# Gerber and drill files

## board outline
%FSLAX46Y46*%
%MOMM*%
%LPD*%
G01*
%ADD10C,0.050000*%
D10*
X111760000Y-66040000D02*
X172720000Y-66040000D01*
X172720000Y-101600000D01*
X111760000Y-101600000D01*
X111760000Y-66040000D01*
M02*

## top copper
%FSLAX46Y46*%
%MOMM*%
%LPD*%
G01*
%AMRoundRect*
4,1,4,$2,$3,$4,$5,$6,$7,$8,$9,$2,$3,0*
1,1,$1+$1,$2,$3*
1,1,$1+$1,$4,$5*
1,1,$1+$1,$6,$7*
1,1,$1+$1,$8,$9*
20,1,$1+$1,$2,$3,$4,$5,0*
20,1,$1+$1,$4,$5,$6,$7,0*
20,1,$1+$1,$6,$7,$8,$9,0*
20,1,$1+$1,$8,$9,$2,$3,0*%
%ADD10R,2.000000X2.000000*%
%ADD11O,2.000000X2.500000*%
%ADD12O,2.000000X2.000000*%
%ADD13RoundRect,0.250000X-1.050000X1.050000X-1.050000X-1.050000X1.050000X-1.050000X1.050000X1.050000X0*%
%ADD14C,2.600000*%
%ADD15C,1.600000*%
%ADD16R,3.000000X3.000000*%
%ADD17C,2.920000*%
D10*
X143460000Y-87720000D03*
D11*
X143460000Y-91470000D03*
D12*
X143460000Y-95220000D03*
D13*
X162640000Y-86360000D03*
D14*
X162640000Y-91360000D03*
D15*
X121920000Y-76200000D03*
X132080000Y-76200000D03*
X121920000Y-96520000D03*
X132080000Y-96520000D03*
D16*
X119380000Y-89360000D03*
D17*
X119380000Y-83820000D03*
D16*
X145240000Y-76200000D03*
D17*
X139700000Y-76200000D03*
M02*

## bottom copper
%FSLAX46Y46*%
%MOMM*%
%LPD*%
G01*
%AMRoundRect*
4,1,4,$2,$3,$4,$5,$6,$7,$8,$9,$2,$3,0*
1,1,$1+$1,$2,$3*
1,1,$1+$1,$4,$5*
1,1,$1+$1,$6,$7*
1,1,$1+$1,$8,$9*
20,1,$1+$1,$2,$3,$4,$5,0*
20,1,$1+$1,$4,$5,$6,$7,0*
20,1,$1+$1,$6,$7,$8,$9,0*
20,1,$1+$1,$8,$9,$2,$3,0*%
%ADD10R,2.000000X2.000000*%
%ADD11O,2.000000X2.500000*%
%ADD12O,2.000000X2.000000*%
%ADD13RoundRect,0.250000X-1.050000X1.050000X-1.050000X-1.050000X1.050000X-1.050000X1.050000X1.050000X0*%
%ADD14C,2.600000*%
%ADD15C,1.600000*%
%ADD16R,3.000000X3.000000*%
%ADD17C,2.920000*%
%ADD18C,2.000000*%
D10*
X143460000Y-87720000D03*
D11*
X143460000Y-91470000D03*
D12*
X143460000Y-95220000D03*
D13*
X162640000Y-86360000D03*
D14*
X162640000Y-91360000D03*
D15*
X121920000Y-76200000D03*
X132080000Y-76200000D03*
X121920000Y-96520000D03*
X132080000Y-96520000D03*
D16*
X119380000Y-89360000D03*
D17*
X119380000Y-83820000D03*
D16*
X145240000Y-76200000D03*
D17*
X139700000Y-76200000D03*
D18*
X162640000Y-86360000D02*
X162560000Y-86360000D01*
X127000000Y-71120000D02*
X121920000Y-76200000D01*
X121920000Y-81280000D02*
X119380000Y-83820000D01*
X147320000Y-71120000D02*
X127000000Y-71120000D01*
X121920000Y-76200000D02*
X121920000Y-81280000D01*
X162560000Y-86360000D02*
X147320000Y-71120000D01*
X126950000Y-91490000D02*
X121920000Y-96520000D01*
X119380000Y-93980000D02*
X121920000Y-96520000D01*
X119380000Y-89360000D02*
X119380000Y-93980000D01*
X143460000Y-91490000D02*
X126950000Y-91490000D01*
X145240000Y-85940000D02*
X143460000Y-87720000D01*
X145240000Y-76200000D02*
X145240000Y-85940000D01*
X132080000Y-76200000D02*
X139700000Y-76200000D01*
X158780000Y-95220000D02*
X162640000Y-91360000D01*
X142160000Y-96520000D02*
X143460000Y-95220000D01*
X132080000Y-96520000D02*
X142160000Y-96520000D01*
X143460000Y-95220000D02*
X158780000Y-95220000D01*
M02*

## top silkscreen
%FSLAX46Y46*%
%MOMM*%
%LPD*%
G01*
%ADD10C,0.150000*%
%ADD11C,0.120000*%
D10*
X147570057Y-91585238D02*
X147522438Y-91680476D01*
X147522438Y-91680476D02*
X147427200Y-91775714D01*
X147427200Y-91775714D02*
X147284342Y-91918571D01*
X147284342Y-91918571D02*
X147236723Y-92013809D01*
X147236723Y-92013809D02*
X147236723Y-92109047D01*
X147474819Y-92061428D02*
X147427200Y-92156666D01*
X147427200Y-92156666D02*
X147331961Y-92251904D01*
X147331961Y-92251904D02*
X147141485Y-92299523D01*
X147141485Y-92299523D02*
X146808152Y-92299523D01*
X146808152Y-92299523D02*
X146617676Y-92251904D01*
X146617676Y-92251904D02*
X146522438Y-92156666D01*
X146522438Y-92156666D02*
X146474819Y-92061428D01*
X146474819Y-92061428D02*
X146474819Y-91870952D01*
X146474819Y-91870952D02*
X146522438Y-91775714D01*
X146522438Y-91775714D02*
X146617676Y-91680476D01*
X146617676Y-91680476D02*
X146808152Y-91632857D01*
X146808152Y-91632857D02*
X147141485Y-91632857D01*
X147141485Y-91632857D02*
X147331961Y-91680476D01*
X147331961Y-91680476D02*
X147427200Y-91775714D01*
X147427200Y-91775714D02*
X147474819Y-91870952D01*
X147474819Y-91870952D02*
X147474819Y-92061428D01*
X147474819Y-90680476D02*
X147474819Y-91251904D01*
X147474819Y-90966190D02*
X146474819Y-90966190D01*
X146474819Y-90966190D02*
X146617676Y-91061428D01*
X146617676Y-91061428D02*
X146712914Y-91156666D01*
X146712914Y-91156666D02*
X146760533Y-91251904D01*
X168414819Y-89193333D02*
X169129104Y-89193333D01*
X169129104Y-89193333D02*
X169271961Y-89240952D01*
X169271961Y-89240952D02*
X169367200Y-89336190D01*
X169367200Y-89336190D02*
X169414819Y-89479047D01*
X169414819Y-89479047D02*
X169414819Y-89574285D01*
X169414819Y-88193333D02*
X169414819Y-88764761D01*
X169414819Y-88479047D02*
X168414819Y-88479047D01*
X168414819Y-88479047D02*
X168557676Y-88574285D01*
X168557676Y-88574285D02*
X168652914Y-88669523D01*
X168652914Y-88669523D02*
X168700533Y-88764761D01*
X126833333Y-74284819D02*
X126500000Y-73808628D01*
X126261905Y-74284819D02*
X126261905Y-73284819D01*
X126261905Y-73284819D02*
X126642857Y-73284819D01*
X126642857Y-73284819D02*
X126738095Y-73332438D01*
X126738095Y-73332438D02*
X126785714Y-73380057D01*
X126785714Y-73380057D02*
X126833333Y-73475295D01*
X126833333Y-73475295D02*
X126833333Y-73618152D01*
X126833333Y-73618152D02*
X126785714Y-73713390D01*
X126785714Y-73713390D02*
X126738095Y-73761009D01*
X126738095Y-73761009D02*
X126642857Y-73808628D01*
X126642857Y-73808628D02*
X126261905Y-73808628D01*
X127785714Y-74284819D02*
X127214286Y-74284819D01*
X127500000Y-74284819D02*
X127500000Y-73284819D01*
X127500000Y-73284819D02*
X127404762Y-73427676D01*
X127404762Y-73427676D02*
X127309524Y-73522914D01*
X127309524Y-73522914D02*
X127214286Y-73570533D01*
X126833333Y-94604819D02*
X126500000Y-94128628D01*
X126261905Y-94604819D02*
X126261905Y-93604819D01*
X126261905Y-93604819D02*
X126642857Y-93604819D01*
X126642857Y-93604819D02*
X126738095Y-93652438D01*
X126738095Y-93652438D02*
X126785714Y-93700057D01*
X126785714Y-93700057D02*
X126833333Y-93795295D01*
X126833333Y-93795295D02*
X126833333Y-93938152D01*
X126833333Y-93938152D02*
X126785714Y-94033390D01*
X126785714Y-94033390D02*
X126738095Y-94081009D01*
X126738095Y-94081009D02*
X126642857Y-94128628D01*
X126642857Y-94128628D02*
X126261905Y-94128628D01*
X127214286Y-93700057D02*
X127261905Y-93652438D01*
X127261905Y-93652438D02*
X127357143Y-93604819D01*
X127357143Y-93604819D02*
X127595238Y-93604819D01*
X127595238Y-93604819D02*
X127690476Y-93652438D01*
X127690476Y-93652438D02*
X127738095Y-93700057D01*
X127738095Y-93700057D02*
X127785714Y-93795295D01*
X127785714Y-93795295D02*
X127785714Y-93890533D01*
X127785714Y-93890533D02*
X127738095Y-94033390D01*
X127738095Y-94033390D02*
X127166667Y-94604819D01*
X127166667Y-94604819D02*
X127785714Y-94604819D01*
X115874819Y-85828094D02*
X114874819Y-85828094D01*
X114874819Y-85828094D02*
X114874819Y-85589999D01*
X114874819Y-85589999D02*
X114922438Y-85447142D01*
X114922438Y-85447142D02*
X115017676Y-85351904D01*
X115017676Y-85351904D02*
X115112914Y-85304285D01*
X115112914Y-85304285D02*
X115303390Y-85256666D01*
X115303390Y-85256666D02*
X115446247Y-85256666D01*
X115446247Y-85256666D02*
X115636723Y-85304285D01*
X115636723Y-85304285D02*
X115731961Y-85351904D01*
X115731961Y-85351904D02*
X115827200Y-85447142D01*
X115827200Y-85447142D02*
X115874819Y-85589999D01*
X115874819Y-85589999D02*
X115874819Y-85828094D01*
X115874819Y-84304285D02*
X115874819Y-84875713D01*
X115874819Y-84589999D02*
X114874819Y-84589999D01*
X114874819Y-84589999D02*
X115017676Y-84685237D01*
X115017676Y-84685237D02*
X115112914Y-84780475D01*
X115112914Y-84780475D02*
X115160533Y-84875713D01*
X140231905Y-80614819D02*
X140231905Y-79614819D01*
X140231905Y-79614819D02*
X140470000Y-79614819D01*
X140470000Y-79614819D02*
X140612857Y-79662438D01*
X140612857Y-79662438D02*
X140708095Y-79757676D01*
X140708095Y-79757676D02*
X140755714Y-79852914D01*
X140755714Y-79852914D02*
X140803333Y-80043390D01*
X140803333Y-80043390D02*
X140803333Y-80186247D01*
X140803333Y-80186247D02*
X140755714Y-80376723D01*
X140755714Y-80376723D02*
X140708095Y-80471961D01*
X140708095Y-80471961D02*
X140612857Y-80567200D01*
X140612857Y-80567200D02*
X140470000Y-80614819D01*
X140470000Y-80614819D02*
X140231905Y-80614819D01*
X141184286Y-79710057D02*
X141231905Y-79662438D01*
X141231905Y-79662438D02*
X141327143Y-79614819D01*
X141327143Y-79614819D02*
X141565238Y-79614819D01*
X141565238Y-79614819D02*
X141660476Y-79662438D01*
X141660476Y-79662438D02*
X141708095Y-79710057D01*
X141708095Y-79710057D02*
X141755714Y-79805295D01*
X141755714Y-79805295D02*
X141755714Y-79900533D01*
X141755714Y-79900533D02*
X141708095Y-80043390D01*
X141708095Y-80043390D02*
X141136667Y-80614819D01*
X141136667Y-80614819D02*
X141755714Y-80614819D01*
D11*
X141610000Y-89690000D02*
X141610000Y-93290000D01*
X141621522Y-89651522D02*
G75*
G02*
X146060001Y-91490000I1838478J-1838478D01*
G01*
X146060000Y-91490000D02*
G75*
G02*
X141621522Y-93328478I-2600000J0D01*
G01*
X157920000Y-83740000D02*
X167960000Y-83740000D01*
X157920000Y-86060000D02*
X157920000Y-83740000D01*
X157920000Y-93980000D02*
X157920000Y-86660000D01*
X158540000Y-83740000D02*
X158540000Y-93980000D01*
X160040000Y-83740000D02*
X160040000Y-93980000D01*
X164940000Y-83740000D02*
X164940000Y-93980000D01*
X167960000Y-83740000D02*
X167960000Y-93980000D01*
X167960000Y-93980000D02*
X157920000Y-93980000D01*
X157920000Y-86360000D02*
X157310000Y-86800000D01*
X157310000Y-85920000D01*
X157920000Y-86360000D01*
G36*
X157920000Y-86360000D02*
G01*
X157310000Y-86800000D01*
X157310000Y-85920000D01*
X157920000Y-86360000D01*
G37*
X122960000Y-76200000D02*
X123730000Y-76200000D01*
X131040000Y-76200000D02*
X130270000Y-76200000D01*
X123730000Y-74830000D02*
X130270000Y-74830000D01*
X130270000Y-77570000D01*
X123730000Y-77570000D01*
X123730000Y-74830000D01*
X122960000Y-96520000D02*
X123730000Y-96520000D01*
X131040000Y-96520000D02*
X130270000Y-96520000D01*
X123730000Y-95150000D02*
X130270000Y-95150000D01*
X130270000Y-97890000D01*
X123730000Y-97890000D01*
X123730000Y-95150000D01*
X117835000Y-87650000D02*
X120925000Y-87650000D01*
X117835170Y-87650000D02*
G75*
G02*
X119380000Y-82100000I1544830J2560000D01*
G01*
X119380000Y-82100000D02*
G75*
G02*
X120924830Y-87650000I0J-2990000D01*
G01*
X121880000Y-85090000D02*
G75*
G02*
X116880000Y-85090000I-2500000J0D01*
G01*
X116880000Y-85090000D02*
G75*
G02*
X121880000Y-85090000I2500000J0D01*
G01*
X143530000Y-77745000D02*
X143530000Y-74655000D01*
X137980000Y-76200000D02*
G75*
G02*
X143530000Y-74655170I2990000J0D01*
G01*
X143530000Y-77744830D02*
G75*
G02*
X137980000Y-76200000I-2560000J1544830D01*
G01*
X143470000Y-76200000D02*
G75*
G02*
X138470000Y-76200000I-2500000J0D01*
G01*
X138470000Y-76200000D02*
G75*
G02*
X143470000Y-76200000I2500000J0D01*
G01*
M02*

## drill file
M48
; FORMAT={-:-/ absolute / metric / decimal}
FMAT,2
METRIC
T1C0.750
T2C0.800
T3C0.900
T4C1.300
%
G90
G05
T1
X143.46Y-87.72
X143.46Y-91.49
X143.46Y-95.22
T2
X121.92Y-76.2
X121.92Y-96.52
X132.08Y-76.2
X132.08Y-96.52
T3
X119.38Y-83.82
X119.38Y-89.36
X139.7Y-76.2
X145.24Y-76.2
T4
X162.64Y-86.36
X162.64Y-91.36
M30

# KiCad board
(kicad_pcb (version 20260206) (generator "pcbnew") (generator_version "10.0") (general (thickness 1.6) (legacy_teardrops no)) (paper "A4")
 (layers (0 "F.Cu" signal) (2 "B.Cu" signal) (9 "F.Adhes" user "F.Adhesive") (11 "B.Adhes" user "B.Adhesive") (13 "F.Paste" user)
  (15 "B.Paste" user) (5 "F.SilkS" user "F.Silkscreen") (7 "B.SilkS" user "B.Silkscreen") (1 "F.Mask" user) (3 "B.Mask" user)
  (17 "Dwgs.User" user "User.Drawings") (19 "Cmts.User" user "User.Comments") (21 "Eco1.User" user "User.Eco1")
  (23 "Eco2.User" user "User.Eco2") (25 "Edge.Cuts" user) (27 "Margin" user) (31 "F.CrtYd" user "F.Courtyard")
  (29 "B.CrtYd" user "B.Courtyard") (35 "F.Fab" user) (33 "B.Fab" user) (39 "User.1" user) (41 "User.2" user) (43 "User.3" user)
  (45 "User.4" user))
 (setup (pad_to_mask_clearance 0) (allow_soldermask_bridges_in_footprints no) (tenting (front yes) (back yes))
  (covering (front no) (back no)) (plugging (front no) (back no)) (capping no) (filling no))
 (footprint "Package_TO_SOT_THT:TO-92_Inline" (layer "F.Cu") (at 143.46 90.22 -90)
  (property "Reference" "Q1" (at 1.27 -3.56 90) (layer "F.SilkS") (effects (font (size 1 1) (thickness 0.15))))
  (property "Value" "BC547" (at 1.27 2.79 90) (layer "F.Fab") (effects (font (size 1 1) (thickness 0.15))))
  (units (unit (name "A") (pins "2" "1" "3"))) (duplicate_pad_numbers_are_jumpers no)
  (fp_line (start -0.53 1.85) (end 3.07 1.85) (stroke (width 0.12) (type solid)) (layer "F.SilkS"))
  (fp_arc (start -0.568478 1.838478) (mid -1.132087 -0.994977) (end 1.27 -2.6) (stroke (width 0.12) (type solid)) (layer "F.SilkS"))
  (fp_arc (start 1.27 -2.6) (mid 3.672087 -0.994977) (end 3.108478 1.838478) (stroke (width 0.12) (type solid)) (layer "F.SilkS"))
  (pad "1" thru_hole rect (at -2.5 0 270) (size 2 2) (drill 0.75) (layers "*.Cu" "*.Mask") (remove_unused_layers no) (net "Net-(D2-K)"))
  (pad "2" thru_hole oval (at 1.27 0 270) (size 2.5 2) (drill 0.75 (offset -0.02 0)) (layers "*.Cu" "*.Mask") (remove_unused_layers no)
   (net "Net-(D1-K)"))
  (pad "3" thru_hole oval (at 5 0 270) (size 2 2) (drill 0.75) (layers "*.Cu" "*.Mask") (remove_unused_layers no) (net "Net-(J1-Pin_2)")))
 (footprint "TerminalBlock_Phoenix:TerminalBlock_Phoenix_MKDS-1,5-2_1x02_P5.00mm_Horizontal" (layer "F.Cu") (at 162.64 86.36 -90)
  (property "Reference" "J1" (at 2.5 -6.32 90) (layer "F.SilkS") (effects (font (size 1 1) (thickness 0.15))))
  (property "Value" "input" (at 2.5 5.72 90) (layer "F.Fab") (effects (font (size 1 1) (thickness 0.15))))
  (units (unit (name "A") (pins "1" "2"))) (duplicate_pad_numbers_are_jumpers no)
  (fp_line (start -2.62 4.72) (end -2.62 -5.32) (stroke (width 0.12) (type solid)) (layer "F.SilkS"))
  (fp_line (start -0.3 4.72) (end -2.62 4.72) (stroke (width 0.12) (type solid)) (layer "F.SilkS"))
  (fp_line (start 7.62 4.72) (end 0.3 4.72) (stroke (width 0.12) (type solid)) (layer "F.SilkS"))
  (fp_line (start -2.62 4.1) (end 7.62 4.1) (stroke (width 0.12) (type solid)) (layer "F.SilkS"))
  (fp_line (start -2.62 2.6) (end 7.62 2.6) (stroke (width 0.12) (type solid)) (layer "F.SilkS"))
  (fp_line (start -2.62 -2.3) (end 7.62 -2.3) (stroke (width 0.12) (type solid)) (layer "F.SilkS"))
  (fp_line (start -2.62 -5.32) (end 7.62 -5.32) (stroke (width 0.12) (type solid)) (layer "F.SilkS"))
  (fp_line (start 7.62 -5.32) (end 7.62 4.72) (stroke (width 0.12) (type solid)) (layer "F.SilkS"))
  (fp_poly (pts (xy 0 4.72) (xy 0.44 5.33) (xy -0.44 5.33)) (stroke (width 0.12) (type solid)) (fill yes) (layer "F.SilkS"))
  (pad "1" thru_hole roundrect (at 0 0 270) (size 2.6 2.6) (drill 1.3) (layers "*.Cu" "*.Mask") (remove_unused_layers no)
   (roundrect_rratio 0.096154) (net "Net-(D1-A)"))
  (pad "2" thru_hole circle (at 5 0 270) (size 2.6 2.6) (drill 1.3) (layers "*.Cu" "*.Mask") (remove_unused_layers no)
   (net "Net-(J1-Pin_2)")))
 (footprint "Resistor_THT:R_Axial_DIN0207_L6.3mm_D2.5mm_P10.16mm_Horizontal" (layer "F.Cu") (at 121.92 76.2)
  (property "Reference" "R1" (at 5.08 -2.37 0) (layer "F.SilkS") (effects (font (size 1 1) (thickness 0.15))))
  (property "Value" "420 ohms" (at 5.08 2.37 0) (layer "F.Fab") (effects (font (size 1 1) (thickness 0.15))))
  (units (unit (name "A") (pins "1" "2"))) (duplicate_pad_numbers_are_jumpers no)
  (fp_line (start 1.04 0) (end 1.81 0) (stroke (width 0.12) (type solid)) (layer "F.SilkS"))
  (fp_line (start 9.12 0) (end 8.35 0) (stroke (width 0.12) (type solid)) (layer "F.SilkS"))
  (fp_rect (start 1.81 -1.37) (end 8.35 1.37) (stroke (width 0.12) (type solid)) (fill no) (layer "F.SilkS"))
  (pad "1" thru_hole circle (at 0 0) (size 1.6 1.6) (drill 0.8) (layers "*.Cu" "*.Mask") (remove_unused_layers no) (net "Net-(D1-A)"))
  (pad "2" thru_hole circle (at 10.16 0) (size 1.6 1.6) (drill 0.8) (layers "*.Cu" "*.Mask") (remove_unused_layers no) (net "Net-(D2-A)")))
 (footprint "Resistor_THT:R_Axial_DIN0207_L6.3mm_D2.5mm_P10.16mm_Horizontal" (layer "F.Cu") (at 121.92 96.52)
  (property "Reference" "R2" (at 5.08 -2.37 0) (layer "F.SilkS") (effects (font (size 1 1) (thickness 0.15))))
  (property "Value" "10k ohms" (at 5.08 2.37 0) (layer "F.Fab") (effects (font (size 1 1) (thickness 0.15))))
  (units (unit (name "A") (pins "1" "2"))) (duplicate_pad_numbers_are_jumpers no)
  (fp_line (start 1.04 0) (end 1.81 0) (stroke (width 0.12) (type solid)) (layer "F.SilkS"))
  (fp_line (start 9.12 0) (end 8.35 0) (stroke (width 0.12) (type solid)) (layer "F.SilkS"))
  (fp_rect (start 1.81 -1.37) (end 8.35 1.37) (stroke (width 0.12) (type solid)) (fill no) (layer "F.SilkS"))
  (pad "1" thru_hole circle (at 0 0) (size 1.6 1.6) (drill 0.8) (layers "*.Cu" "*.Mask") (remove_unused_layers no) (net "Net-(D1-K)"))
  (pad "2" thru_hole circle (at 10.16 0) (size 1.6 1.6) (drill 0.8) (layers "*.Cu" "*.Mask") (remove_unused_layers no)
   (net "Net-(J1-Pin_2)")))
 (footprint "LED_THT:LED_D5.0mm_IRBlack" (layer "F.Cu") (at 119.38 86.36 90)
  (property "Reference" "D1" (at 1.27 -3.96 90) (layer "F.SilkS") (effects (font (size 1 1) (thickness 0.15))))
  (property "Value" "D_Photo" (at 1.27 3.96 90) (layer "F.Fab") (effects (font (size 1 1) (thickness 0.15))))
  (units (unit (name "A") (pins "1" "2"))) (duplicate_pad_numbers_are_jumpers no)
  (fp_line (start -1.29 -1.545) (end -1.29 1.545) (stroke (width 0.12) (type solid)) (layer "F.SilkS"))
  (fp_arc (start -1.29 -1.54483) (mid 2.071779 -2.880495) (end 4.26 0) (stroke (width 0.12) (type solid)) (layer "F.SilkS"))
  (fp_arc (start 4.26 0) (mid 2.071779 2.880495) (end -1.29 1.54483) (stroke (width 0.12) (type solid)) (layer "F.SilkS"))
  (fp_circle (center 1.27 0) (end 3.77 0) (stroke (width 0.12) (type solid)) (fill no) (layer "F.SilkS"))
  (pad "1" thru_hole rect (at -3 0 90) (size 3 3) (drill 0.9) (layers "*.Cu" "*.Mask") (remove_unused_layers no) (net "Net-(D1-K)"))
  (pad "2" thru_hole circle (at 2.54 0 90) (size 2.92 2.92) (drill 0.9) (layers "*.Cu" "*.Mask") (remove_unused_layers no)
   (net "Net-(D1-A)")))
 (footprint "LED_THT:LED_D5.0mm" (layer "F.Cu") (at 142.24 76.2 180)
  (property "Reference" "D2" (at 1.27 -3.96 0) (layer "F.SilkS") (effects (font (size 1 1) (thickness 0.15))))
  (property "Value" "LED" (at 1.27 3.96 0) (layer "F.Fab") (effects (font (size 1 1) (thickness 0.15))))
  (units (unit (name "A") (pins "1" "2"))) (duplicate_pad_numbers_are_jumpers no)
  (fp_line (start -1.29 -1.545) (end -1.29 1.545) (stroke (width 0.12) (type solid)) (layer "F.SilkS"))
  (fp_arc (start 4.26 0) (mid 2.071779 2.880495) (end -1.29 1.54483) (stroke (width 0.12) (type solid)) (layer "F.SilkS"))
  (fp_arc (start -1.29 -1.54483) (mid 2.071779 -2.880495) (end 4.26 0) (stroke (width 0.12) (type solid)) (layer "F.SilkS"))
  (fp_circle (center 1.27 0) (end 3.77 0) (stroke (width 0.12) (type solid)) (fill no) (layer "F.SilkS"))
  (pad "1" thru_hole rect (at -3 0 180) (size 3 3) (drill 0.9) (layers "*.Cu" "*.Mask") (remove_unused_layers no) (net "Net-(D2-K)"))
  (pad "2" thru_hole circle (at 2.54 0 180) (size 2.92 2.92) (drill 0.9) (layers "*.Cu" "*.Mask") (remove_unused_layers no)
   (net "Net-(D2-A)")))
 (gr_rect (start 111.76 66.04) (end 172.72 101.6) (stroke (width 0.05) (type default)) (fill no) (layer "Edge.Cuts"))
 (segment (start 162.64 86.36) (end 162.56 86.36) (width 2) (layer "B.Cu") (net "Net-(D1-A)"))
 (segment (start 127 71.12) (end 121.92 76.2) (width 2) (layer "B.Cu") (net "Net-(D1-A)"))
 (segment (start 121.92 81.28) (end 119.38 83.82) (width 2) (layer "B.Cu") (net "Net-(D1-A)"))
 (segment (start 147.32 71.12) (end 127 71.12) (width 2) (layer "B.Cu") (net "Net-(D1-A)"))
 (segment (start 121.92 76.2) (end 121.92 81.28) (width 2) (layer "B.Cu") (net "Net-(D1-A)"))
 (segment (start 162.56 86.36) (end 147.32 71.12) (width 2) (layer "B.Cu") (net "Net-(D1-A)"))
 (segment (start 126.95 91.49) (end 121.92 96.52) (width 2) (layer "B.Cu") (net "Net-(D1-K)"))
 (segment (start 119.38 93.98) (end 121.92 96.52) (width 2) (layer "B.Cu") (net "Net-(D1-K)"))
 (segment (start 119.38 89.36) (end 119.38 93.98) (width 2) (layer "B.Cu") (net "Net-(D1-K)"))
 (segment (start 143.46 91.49) (end 126.95 91.49) (width 2) (layer "B.Cu") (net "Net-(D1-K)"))
 (segment (start 145.24 85.94) (end 143.46 87.72) (width 2) (layer "B.Cu") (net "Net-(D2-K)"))
 (segment (start 145.24 76.2) (end 145.24 85.94) (width 2) (layer "B.Cu") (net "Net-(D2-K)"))
 (segment (start 132.08 76.2) (end 139.7 76.2) (width 2) (layer "B.Cu") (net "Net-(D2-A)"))
 (segment (start 158.78 95.22) (end 162.64 91.36) (width 2) (layer "B.Cu") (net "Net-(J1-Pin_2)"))
 (segment (start 142.16 96.52) (end 143.46 95.22) (width 2) (layer "B.Cu") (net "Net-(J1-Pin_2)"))
 (segment (start 132.08 96.52) (end 142.16 96.52) (width 2) (layer "B.Cu") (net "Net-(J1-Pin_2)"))
 (segment (start 143.46 95.22) (end 158.78 95.22) (width 2) (layer "B.Cu") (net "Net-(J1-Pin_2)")))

